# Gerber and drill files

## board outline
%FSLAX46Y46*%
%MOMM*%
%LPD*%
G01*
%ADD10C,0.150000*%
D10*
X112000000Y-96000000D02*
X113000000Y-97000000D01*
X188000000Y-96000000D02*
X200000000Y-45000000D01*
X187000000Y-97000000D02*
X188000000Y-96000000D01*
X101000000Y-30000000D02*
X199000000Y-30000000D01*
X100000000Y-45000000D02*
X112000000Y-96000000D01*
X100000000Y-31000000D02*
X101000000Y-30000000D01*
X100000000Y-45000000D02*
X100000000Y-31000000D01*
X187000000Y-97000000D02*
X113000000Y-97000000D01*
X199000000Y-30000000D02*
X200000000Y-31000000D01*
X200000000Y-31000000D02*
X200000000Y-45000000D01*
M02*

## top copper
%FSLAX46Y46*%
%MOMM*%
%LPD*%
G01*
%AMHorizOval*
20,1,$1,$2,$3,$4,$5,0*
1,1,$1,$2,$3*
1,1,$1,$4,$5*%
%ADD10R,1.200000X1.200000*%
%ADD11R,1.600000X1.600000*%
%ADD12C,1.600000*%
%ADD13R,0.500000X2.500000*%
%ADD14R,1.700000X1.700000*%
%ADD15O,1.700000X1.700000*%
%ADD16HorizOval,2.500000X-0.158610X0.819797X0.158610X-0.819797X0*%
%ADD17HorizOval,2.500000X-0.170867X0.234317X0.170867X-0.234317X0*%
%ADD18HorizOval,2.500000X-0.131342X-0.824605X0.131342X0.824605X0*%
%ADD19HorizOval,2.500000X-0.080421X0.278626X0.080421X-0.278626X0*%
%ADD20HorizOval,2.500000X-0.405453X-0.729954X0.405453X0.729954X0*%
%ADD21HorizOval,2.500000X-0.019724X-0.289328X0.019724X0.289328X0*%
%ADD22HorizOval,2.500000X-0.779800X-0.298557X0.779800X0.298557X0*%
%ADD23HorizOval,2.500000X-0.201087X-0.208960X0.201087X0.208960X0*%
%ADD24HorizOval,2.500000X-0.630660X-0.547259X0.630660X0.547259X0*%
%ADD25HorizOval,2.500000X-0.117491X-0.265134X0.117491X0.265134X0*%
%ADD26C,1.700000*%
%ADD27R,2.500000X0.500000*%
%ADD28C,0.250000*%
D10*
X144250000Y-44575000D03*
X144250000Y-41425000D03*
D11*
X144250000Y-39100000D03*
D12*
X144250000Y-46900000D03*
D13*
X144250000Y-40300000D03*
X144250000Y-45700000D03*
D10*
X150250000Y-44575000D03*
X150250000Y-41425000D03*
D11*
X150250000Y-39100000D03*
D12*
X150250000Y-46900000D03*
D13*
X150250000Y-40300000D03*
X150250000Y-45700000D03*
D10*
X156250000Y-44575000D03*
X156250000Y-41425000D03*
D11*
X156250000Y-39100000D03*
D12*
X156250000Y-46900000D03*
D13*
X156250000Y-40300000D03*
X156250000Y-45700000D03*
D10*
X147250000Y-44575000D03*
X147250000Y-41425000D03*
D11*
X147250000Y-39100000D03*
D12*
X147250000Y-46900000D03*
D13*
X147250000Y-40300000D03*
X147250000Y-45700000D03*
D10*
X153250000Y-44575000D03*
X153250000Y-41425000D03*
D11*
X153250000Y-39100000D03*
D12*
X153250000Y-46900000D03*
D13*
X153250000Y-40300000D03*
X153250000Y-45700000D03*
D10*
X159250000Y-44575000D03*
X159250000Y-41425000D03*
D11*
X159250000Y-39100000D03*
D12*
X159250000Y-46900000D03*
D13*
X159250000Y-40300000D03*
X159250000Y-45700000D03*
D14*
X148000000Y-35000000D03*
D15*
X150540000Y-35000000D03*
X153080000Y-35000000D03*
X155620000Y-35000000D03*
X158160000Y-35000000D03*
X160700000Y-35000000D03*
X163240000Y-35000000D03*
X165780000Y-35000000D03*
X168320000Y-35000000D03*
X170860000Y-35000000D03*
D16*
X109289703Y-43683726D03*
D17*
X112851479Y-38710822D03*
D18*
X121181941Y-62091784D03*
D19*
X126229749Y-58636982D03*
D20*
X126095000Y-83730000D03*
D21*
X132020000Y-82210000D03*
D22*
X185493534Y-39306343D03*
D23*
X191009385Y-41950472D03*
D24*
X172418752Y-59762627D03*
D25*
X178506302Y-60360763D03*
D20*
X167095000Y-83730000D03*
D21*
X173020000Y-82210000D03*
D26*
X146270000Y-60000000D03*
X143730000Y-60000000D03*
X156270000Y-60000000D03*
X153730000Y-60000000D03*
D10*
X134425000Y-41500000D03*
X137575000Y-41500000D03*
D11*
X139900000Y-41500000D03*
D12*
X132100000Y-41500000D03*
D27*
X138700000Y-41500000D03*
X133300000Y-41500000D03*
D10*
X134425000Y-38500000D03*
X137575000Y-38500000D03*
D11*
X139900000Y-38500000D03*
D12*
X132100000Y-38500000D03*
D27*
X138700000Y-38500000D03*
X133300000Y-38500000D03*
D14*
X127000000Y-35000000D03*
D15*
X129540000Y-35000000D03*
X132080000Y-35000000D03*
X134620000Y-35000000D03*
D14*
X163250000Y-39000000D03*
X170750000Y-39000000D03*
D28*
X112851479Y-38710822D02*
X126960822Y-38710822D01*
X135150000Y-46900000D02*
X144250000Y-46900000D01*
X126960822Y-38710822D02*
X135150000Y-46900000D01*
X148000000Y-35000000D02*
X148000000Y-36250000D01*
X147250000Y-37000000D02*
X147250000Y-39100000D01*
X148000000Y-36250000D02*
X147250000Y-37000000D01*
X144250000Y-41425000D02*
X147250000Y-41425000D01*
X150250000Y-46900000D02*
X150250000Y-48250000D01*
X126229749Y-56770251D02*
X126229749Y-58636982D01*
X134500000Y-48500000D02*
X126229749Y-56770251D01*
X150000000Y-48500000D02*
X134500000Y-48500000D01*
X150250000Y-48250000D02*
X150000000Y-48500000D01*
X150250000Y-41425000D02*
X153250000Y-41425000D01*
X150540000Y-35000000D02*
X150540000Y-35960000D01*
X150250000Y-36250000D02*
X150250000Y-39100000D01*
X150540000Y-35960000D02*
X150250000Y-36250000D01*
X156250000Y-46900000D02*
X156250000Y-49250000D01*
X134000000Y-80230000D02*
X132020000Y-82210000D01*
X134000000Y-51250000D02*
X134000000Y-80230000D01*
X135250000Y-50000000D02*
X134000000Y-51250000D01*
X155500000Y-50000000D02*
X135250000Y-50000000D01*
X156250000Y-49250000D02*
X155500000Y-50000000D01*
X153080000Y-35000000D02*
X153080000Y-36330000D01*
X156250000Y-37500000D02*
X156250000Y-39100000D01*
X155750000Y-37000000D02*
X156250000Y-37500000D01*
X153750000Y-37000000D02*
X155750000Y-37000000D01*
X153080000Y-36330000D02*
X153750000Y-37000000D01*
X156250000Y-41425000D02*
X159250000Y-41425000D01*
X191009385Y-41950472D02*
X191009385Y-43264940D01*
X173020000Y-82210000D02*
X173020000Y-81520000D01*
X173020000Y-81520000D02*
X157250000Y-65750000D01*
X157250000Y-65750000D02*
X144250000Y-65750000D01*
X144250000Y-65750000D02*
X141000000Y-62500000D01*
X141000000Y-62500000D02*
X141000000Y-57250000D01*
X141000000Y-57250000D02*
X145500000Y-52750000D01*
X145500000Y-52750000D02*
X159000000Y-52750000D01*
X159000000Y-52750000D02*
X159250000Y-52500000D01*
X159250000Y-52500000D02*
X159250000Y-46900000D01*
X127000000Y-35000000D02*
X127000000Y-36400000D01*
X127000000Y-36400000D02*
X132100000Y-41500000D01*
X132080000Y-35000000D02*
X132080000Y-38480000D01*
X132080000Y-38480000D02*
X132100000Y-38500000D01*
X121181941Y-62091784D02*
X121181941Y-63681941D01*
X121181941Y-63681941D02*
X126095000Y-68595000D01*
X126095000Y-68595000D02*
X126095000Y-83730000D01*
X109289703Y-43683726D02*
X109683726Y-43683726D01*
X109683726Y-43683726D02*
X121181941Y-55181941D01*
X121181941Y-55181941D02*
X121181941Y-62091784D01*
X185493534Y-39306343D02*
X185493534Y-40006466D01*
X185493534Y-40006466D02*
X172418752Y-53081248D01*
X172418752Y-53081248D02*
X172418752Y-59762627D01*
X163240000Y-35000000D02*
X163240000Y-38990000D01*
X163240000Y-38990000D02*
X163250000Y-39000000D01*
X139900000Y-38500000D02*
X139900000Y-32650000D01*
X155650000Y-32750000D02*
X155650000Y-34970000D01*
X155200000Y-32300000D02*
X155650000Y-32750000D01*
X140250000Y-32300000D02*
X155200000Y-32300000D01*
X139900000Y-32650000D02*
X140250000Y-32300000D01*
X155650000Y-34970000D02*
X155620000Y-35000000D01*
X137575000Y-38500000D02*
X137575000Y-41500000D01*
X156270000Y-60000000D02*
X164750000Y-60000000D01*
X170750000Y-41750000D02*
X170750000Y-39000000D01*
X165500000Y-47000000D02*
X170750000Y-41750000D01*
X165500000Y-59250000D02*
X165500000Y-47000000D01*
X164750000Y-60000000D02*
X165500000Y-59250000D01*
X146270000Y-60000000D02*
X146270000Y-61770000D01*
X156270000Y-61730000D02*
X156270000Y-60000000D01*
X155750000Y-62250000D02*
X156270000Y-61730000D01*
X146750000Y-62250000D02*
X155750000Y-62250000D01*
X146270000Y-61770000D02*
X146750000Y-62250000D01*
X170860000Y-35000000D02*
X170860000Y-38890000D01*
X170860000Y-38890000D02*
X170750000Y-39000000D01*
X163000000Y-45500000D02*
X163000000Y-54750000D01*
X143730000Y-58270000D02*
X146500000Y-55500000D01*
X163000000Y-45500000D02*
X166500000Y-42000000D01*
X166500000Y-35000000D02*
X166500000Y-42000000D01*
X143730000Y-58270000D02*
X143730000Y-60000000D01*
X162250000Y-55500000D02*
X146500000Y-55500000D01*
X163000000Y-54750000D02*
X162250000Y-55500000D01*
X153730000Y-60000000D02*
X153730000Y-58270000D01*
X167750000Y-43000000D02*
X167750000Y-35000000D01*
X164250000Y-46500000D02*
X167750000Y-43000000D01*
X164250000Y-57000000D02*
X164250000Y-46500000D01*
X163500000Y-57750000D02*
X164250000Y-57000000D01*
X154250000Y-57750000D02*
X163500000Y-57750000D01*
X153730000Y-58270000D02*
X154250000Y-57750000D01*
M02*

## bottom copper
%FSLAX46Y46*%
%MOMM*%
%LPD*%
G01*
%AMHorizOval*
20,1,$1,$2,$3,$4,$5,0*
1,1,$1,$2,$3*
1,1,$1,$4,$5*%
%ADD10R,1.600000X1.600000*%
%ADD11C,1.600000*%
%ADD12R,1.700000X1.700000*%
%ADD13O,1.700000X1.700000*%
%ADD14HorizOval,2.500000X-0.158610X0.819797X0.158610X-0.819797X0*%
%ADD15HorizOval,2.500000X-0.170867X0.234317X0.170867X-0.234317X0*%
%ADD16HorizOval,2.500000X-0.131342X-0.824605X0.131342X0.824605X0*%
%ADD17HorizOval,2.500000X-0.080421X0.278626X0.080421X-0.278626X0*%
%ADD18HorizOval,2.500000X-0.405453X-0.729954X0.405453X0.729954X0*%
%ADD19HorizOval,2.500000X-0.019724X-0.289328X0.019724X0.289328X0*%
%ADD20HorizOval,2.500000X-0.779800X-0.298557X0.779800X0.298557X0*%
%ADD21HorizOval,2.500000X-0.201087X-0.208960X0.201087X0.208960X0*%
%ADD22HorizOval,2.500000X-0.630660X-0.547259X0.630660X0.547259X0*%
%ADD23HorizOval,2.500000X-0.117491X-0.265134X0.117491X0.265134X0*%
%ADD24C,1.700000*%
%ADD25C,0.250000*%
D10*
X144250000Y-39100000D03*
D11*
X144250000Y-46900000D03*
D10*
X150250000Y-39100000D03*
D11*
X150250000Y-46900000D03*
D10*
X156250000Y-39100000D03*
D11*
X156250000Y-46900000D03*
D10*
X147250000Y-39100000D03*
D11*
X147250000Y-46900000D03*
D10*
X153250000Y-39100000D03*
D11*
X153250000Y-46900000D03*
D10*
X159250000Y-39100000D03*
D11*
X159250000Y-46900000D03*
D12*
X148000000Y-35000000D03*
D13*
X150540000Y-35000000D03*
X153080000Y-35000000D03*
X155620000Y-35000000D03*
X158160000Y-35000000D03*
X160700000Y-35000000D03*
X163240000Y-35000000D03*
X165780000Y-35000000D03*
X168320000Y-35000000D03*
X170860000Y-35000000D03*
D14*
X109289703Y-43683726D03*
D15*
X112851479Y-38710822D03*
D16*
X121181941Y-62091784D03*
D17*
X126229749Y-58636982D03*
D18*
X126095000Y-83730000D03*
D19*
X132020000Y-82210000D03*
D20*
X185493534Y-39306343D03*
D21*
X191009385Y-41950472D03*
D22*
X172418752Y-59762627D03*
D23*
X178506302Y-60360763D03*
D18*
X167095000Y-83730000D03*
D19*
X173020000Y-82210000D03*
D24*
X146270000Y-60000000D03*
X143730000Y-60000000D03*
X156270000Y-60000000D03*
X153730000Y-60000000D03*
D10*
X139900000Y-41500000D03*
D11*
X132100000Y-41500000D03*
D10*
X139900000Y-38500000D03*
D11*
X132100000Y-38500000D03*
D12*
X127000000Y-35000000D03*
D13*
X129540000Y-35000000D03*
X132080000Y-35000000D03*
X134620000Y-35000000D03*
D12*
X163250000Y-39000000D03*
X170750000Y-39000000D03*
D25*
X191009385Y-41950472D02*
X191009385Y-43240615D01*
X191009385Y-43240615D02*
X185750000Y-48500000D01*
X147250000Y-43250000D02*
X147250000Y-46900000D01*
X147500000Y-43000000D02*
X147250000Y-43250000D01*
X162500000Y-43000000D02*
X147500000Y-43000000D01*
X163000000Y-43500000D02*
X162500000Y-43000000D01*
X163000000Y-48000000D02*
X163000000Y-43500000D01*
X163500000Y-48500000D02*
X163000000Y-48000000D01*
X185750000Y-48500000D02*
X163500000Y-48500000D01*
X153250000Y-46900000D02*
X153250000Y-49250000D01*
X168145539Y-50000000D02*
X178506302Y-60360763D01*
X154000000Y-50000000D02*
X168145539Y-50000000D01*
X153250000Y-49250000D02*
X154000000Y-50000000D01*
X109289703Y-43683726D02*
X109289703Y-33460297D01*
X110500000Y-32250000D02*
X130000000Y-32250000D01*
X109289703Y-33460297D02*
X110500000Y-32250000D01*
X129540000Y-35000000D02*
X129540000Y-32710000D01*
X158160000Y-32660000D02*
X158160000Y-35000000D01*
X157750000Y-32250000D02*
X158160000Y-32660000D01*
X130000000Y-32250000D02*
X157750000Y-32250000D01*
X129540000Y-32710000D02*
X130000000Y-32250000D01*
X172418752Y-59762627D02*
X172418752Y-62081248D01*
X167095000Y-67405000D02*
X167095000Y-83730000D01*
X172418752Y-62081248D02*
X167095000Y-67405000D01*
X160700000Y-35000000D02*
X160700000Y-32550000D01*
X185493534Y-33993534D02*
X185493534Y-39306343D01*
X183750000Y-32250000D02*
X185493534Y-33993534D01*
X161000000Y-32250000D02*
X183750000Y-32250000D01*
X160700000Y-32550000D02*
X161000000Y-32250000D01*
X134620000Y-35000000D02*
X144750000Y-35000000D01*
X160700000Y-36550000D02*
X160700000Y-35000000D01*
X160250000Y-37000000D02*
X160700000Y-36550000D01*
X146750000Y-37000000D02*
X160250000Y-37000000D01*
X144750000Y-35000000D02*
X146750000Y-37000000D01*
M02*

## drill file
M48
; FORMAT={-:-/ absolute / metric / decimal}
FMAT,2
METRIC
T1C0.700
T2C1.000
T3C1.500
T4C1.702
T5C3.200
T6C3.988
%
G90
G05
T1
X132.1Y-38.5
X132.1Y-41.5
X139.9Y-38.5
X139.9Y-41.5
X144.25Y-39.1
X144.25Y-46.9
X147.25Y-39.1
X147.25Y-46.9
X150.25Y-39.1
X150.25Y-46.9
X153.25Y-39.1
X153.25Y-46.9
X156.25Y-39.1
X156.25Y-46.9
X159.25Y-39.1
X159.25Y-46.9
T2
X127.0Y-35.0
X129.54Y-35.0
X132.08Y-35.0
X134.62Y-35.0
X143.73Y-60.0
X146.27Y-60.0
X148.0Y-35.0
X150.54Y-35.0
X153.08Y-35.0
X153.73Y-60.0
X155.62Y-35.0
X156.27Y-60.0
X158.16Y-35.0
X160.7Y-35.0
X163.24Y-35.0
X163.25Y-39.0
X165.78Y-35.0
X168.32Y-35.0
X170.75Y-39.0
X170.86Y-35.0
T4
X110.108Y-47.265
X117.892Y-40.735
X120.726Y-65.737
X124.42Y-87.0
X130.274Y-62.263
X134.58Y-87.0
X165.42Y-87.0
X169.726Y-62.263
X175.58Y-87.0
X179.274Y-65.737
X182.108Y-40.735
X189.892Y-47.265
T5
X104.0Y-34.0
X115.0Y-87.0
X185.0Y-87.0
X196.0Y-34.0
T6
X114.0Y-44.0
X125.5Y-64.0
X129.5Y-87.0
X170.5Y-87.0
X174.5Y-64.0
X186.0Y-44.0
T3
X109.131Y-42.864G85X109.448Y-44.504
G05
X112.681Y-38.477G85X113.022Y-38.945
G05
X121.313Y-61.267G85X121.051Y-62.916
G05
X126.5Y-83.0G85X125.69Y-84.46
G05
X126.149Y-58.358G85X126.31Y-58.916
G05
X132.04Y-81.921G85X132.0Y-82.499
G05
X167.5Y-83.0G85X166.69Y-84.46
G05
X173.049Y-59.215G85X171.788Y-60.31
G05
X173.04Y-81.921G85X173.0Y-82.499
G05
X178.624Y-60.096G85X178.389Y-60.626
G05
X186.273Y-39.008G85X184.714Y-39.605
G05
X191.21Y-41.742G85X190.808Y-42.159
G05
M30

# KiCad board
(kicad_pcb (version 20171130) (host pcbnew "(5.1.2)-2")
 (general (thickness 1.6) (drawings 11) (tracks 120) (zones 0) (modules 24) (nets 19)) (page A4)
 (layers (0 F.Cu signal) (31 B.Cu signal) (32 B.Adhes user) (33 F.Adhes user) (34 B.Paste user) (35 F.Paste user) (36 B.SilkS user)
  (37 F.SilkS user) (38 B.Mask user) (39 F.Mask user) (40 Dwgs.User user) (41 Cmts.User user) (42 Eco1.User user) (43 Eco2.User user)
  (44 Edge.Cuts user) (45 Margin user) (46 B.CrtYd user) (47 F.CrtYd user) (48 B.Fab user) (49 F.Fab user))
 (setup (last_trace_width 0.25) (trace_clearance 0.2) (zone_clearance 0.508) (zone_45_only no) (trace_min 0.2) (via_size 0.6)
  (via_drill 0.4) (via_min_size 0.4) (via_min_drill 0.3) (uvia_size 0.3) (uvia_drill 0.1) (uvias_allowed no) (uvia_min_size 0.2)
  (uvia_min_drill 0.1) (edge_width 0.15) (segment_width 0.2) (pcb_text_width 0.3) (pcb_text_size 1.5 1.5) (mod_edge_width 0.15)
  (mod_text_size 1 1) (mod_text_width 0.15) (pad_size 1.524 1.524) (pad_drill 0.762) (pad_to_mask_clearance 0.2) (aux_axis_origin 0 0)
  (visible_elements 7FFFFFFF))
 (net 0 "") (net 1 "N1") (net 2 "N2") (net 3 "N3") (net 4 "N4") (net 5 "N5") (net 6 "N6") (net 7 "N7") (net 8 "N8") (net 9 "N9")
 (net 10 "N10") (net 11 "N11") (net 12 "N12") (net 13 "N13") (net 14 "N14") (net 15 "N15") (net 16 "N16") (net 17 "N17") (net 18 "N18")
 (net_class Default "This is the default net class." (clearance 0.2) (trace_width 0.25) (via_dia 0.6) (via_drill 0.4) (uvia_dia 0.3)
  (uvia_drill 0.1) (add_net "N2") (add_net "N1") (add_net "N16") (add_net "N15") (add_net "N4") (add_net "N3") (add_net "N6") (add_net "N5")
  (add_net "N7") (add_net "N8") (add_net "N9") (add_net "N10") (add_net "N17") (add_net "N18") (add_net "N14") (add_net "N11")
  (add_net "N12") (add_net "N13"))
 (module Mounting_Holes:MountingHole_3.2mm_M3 (layer F.Cu) (at 115 87)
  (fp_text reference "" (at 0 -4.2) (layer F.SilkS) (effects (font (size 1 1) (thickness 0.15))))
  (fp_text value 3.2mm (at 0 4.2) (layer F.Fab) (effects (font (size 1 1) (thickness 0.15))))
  (pad 1 np_thru_hole circle (at 0 0) (size 3.2 3.2) (drill 3.2) (layers *.Cu *.Mask)))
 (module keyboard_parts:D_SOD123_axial (layer F.Cu) (at 144.25 43 270)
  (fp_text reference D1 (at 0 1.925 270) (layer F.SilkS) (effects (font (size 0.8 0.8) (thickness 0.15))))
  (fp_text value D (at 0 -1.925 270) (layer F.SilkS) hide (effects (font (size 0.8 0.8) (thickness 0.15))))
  (pad 2 smd rect (at 1.575 0 270) (size 1.2 1.2) (layers F.Cu F.Paste F.Mask) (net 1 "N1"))
  (pad 1 smd rect (at -1.575 0 270) (size 1.2 1.2) (layers F.Cu F.Paste F.Mask) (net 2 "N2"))
  (pad 1 thru_hole rect (at -3.9 0 270) (size 1.6 1.6) (drill 0.7) (layers *.Cu *.Mask F.SilkS) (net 2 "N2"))
  (pad 2 thru_hole circle (at 3.9 0 270) (size 1.6 1.6) (drill 0.7) (layers *.Cu *.Mask F.SilkS) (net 1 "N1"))
  (pad 1 smd rect (at -2.7 0 270) (size 2.5 0.5) (layers F.Cu) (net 2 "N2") (solder_mask_margin -999))
  (pad 2 smd rect (at 2.7 0 270) (size 2.5 0.5) (layers F.Cu) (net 1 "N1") (solder_mask_margin -999)))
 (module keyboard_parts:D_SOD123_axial (layer F.Cu) (at 150.25 43 270)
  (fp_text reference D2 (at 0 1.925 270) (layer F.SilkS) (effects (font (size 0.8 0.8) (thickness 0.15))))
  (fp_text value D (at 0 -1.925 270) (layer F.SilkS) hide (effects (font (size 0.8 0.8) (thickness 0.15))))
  (pad 2 smd rect (at 1.575 0 270) (size 1.2 1.2) (layers F.Cu F.Paste F.Mask) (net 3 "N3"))
  (pad 1 smd rect (at -1.575 0 270) (size 1.2 1.2) (layers F.Cu F.Paste F.Mask) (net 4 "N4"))
  (pad 1 thru_hole rect (at -3.9 0 270) (size 1.6 1.6) (drill 0.7) (layers *.Cu *.Mask F.SilkS) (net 4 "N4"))
  (pad 2 thru_hole circle (at 3.9 0 270) (size 1.6 1.6) (drill 0.7) (layers *.Cu *.Mask F.SilkS) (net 3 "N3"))
  (pad 1 smd rect (at -2.7 0 270) (size 2.5 0.5) (layers F.Cu) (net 4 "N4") (solder_mask_margin -999))
  (pad 2 smd rect (at 2.7 0 270) (size 2.5 0.5) (layers F.Cu) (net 3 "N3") (solder_mask_margin -999)))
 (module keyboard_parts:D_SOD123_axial (layer F.Cu) (at 156.25 43 270)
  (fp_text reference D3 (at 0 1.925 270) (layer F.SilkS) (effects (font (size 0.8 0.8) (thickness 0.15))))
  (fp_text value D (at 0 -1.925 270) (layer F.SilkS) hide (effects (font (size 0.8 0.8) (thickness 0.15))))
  (pad 2 smd rect (at 1.575 0 270) (size 1.2 1.2) (layers F.Cu F.Paste F.Mask) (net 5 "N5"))
  (pad 1 smd rect (at -1.575 0 270) (size 1.2 1.2) (layers F.Cu F.Paste F.Mask) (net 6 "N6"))
  (pad 1 thru_hole rect (at -3.9 0 270) (size 1.6 1.6) (drill 0.7) (layers *.Cu *.Mask F.SilkS) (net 6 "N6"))
  (pad 2 thru_hole circle (at 3.9 0 270) (size 1.6 1.6) (drill 0.7) (layers *.Cu *.Mask F.SilkS) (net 5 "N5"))
  (pad 1 smd rect (at -2.7 0 270) (size 2.5 0.5) (layers F.Cu) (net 6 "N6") (solder_mask_margin -999))
  (pad 2 smd rect (at 2.7 0 270) (size 2.5 0.5) (layers F.Cu) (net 5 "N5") (solder_mask_margin -999)))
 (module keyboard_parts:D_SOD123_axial (layer F.Cu) (at 147.25 43 270)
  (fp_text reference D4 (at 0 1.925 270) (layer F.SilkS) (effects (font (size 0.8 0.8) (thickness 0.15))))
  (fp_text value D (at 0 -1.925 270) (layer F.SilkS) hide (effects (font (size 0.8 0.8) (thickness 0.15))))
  (pad 2 smd rect (at 1.575 0 270) (size 1.2 1.2) (layers F.Cu F.Paste F.Mask) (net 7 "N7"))
  (pad 1 smd rect (at -1.575 0 270) (size 1.2 1.2) (layers F.Cu F.Paste F.Mask) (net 2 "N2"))
  (pad 1 thru_hole rect (at -3.9 0 270) (size 1.6 1.6) (drill 0.7) (layers *.Cu *.Mask F.SilkS) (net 2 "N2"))
  (pad 2 thru_hole circle (at 3.9 0 270) (size 1.6 1.6) (drill 0.7) (layers *.Cu *.Mask F.SilkS) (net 7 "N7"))
  (pad 1 smd rect (at -2.7 0 270) (size 2.5 0.5) (layers F.Cu) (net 2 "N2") (solder_mask_margin -999))
  (pad 2 smd rect (at 2.7 0 270) (size 2.5 0.5) (layers F.Cu) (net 7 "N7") (solder_mask_margin -999)))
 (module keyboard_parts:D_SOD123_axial (layer F.Cu) (at 153.25 43 270)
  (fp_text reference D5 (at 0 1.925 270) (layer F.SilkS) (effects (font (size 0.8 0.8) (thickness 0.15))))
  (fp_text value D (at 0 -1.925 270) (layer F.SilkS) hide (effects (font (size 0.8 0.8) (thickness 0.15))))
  (pad 2 smd rect (at 1.575 0 270) (size 1.2 1.2) (layers F.Cu F.Paste F.Mask) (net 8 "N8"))
  (pad 1 smd rect (at -1.575 0 270) (size 1.2 1.2) (layers F.Cu F.Paste F.Mask) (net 4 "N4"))
  (pad 1 thru_hole rect (at -3.9 0 270) (size 1.6 1.6) (drill 0.7) (layers *.Cu *.Mask F.SilkS) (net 4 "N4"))
  (pad 2 thru_hole circle (at 3.9 0 270) (size 1.6 1.6) (drill 0.7) (layers *.Cu *.Mask F.SilkS) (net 8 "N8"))
  (pad 1 smd rect (at -2.7 0 270) (size 2.5 0.5) (layers F.Cu) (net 4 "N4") (solder_mask_margin -999))
  (pad 2 smd rect (at 2.7 0 270) (size 2.5 0.5) (layers F.Cu) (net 8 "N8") (solder_mask_margin -999)))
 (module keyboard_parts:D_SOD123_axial (layer F.Cu) (at 159.25 43 270)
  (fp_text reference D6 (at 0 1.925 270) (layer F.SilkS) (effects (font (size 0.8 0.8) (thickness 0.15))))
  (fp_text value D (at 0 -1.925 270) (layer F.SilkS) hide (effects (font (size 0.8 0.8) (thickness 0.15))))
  (pad 2 smd rect (at 1.575 0 270) (size 1.2 1.2) (layers F.Cu F.Paste F.Mask) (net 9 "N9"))
  (pad 1 smd rect (at -1.575 0 270) (size 1.2 1.2) (layers F.Cu F.Paste F.Mask) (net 6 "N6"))
  (pad 1 thru_hole rect (at -3.9 0 270) (size 1.6 1.6) (drill 0.7) (layers *.Cu *.Mask F.SilkS) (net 6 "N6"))
  (pad 2 thru_hole circle (at 3.9 0 270) (size 1.6 1.6) (drill 0.7) (layers *.Cu *.Mask F.SilkS) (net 9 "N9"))
  (pad 1 smd rect (at -2.7 0 270) (size 2.5 0.5) (layers F.Cu) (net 6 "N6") (solder_mask_margin -999))
  (pad 2 smd rect (at 2.7 0 270) (size 2.5 0.5) (layers F.Cu) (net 9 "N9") (solder_mask_margin -999)))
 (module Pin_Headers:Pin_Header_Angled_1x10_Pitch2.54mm (layer F.Cu) (at 148 35 90)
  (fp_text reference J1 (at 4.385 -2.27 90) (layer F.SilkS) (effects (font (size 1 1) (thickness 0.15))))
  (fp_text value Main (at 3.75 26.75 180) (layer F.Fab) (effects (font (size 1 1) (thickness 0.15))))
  (pad 1 thru_hole rect (at 0 0 90) (size 1.7 1.7) (drill 1) (layers *.Cu *.Mask) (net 2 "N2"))
  (pad 2 thru_hole oval (at 0 2.54 90) (size 1.7 1.7) (drill 1) (layers *.Cu *.Mask) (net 4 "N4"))
  (pad 3 thru_hole oval (at 0 5.08 90) (size 1.7 1.7) (drill 1) (layers *.Cu *.Mask) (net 6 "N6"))
  (pad 4 thru_hole oval (at 0 7.62 90) (size 1.7 1.7) (drill 1) (layers *.Cu *.Mask) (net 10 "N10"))
  (pad 5 thru_hole oval (at 0 10.16 90) (size 1.7 1.7) (drill 1) (layers *.Cu *.Mask) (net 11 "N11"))
  (pad 6 thru_hole oval (at 0 12.7 90) (size 1.7 1.7) (drill 1) (layers *.Cu *.Mask) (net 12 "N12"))
  (pad 7 thru_hole oval (at 0 15.24 90) (size 1.7 1.7) (drill 1) (layers *.Cu *.Mask) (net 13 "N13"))
  (pad 8 thru_hole oval (at 0 17.78 90) (size 1.7 1.7) (drill 1) (layers *.Cu *.Mask) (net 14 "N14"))
  (pad 9 thru_hole oval (at 0 20.32 90) (size 1.7 1.7) (drill 1) (layers *.Cu *.Mask) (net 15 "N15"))
  (pad 10 thru_hole oval (at 0 22.86 90) (size 1.7 1.7) (drill 1) (layers *.Cu *.Mask) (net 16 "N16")))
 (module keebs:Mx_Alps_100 (layer F.Cu) (at 114 44 40)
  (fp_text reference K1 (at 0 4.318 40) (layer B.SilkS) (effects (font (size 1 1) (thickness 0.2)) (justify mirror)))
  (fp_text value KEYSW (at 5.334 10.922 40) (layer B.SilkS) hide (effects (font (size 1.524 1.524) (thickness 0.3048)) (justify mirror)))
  (pad HOLE np_thru_hole circle (at 0 0 40) (size 3.9878 3.9878) (drill 3.9878) (layers *.Cu))
  (pad HOLE np_thru_hole circle (at -5.08 0 40) (size 1.7018 1.7018) (drill 1.7018) (layers *.Cu))
  (pad HOLE np_thru_hole circle (at 5.08 0 40) (size 1.7018 1.7018) (drill 1.7018) (layers *.Cu))
  (pad 1 thru_hole oval (at -3.405 -3.27 10.95) (size 2.5 4.17) (drill oval 1.5 3.17) (layers *.Cu *.Mask F.SilkS) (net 11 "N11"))
  (pad 2 thru_hole oval (at 2.52 -4.79 36.1) (size 2.5 3.08) (drill oval 1.5 2.08) (layers *.Cu *.Mask F.SilkS) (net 1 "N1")))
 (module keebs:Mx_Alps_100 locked (layer F.Cu) (at 125.5 64 20)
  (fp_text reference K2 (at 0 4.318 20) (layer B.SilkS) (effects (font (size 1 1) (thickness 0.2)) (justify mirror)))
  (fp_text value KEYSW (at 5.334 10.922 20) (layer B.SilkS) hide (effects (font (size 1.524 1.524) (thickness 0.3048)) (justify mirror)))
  (pad HOLE np_thru_hole circle (at 0 0 20) (size 3.9878 3.9878) (drill 3.9878) (layers *.Cu))
  (pad HOLE np_thru_hole circle (at -5.08 0 20) (size 1.7018 1.7018) (drill 1.7018) (layers *.Cu))
  (pad HOLE np_thru_hole circle (at 5.08 0 20) (size 1.7018 1.7018) (drill 1.7018) (layers *.Cu))
  (pad 1 thru_hole oval (at -3.405 -3.27 350.95) (size 2.5 4.17) (drill oval 1.5 3.17) (layers *.Cu *.Mask F.SilkS) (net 11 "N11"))
  (pad 2 thru_hole oval (at 2.52 -4.79 16.1) (size 2.5 3.08) (drill oval 1.5 2.08) (layers *.Cu *.Mask F.SilkS) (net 3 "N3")))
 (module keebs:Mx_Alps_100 (layer F.Cu) (at 129.5 87)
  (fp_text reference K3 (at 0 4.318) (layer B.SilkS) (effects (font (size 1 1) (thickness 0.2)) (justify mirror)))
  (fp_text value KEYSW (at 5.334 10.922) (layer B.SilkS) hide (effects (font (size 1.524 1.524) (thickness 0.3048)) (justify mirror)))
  (pad HOLE np_thru_hole circle (at 0 0) (size 3.9878 3.9878) (drill 3.9878) (layers *.Cu))
  (pad HOLE np_thru_hole circle (at -5.08 0) (size 1.7018 1.7018) (drill 1.7018) (layers *.Cu))
  (pad HOLE np_thru_hole circle (at 5.08 0) (size 1.7018 1.7018) (drill 1.7018) (layers *.Cu))
  (pad 1 thru_hole oval (at -3.405 -3.27 330.95) (size 2.5 4.17) (drill oval 1.5 3.17) (layers *.Cu *.Mask F.SilkS) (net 11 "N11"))
  (pad 2 thru_hole oval (at 2.52 -4.79 356.1) (size 2.5 3.08) (drill oval 1.5 2.08) (layers *.Cu *.Mask F.SilkS) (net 5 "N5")))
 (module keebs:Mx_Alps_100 (layer F.Cu) (at 186 44 320)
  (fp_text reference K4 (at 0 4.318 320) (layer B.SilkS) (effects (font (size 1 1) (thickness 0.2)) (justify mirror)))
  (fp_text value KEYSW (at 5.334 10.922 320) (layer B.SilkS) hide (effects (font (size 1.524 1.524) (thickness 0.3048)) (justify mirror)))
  (pad HOLE np_thru_hole circle (at 0 0 320) (size 3.9878 3.9878) (drill 3.9878) (layers *.Cu))
  (pad HOLE np_thru_hole circle (at -5.08 0 320) (size 1.7018 1.7018) (drill 1.7018) (layers *.Cu))
  (pad HOLE np_thru_hole circle (at 5.08 0 320) (size 1.7018 1.7018) (drill 1.7018) (layers *.Cu))
  (pad 1 thru_hole oval (at -3.405 -3.27 290.95) (size 2.5 4.17) (drill oval 1.5 3.17) (layers *.Cu *.Mask F.SilkS) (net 12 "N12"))
  (pad 2 thru_hole oval (at 2.52 -4.79 316.1) (size 2.5 3.08) (drill oval 1.5 2.08) (layers *.Cu *.Mask F.SilkS) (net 7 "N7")))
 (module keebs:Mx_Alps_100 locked (layer F.Cu) (at 174.5 64 340)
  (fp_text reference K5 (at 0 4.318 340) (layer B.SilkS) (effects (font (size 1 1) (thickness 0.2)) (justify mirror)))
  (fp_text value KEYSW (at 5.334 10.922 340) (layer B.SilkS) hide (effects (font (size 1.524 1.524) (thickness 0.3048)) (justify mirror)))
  (pad HOLE np_thru_hole circle (at 0 0 340) (size 3.9878 3.9878) (drill 3.9878) (layers *.Cu))
  (pad HOLE np_thru_hole circle (at -5.08 0 340) (size 1.7018 1.7018) (drill 1.7018) (layers *.Cu))
  (pad HOLE np_thru_hole circle (at 5.08 0 340) (size 1.7018 1.7018) (drill 1.7018) (layers *.Cu))
  (pad 1 thru_hole oval (at -3.405 -3.27 310.95) (size 2.5 4.17) (drill oval 1.5 3.17) (layers *.Cu *.Mask F.SilkS) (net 12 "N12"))
  (pad 2 thru_hole oval (at 2.52 -4.79 336.1) (size 2.5 3.08) (drill oval 1.5 2.08) (layers *.Cu *.Mask F.SilkS) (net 8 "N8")))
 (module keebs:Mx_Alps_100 (layer F.Cu) (at 170.5 87)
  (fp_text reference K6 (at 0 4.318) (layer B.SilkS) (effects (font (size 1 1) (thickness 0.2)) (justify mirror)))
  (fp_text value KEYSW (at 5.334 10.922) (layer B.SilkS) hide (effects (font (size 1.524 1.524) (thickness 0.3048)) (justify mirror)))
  (pad HOLE np_thru_hole circle (at 0 0) (size 3.9878 3.9878) (drill 3.9878) (layers *.Cu))
  (pad HOLE np_thru_hole circle (at -5.08 0) (size 1.7018 1.7018) (drill 1.7018) (layers *.Cu))
  (pad HOLE np_thru_hole circle (at 5.08 0) (size 1.7018 1.7018) (drill 1.7018) (layers *.Cu))
  (pad 1 thru_hole oval (at -3.405 -3.27 330.95) (size 2.5 4.17) (drill oval 1.5 3.17) (layers *.Cu *.Mask F.SilkS) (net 12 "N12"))
  (pad 2 thru_hole oval (at 2.52 -4.79 356.1) (size 2.5 3.08) (drill oval 1.5 2.08) (layers *.Cu *.Mask F.SilkS) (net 9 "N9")))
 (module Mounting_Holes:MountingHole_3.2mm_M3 (layer F.Cu) (at 196 34)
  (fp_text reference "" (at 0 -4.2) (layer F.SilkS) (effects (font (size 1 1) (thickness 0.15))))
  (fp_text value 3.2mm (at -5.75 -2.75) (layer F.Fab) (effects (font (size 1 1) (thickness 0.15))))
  (pad 1 np_thru_hole circle (at 0 0) (size 3.2 3.2) (drill 3.2) (layers *.Cu *.Mask)))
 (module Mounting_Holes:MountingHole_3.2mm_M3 (layer F.Cu) (at 185 87)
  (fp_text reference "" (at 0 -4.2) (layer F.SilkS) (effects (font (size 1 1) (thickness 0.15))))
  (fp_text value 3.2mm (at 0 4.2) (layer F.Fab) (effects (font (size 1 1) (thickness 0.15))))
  (pad 1 np_thru_hole circle (at 0 0) (size 3.2 3.2) (drill 3.2) (layers *.Cu *.Mask)))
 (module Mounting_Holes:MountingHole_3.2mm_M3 (layer F.Cu) (at 104 34)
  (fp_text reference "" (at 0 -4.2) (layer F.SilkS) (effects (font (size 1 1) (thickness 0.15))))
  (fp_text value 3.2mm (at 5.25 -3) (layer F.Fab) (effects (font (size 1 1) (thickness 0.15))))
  (pad 1 np_thru_hole circle (at 0 0) (size 3.2 3.2) (drill 3.2) (layers *.Cu *.Mask)))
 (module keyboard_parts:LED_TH (layer F.Cu) (at 145 60 180)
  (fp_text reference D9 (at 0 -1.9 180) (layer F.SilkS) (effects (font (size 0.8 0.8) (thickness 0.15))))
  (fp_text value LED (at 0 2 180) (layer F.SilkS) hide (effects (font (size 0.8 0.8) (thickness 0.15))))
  (pad 1 thru_hole circle (at -1.27 0 180) (size 1.7 1.7) (drill 1) (layers *.Cu *.Mask F.SilkS) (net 16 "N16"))
  (pad 2 thru_hole circle (at 1.27 0 180) (size 1.7 1.7) (drill 1) (layers *.Cu *.Mask F.SilkS) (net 14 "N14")))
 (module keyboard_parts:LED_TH (layer F.Cu) (at 155 60 180)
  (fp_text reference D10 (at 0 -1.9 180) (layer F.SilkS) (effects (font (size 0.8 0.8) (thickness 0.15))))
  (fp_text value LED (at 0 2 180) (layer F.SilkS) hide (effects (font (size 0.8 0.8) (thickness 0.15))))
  (pad 1 thru_hole circle (at -1.27 0 180) (size 1.7 1.7) (drill 1) (layers *.Cu *.Mask F.SilkS) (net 16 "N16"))
  (pad 2 thru_hole circle (at 1.27 0 180) (size 1.7 1.7) (drill 1) (layers *.Cu *.Mask F.SilkS) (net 15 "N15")))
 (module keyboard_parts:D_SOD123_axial (layer F.Cu) (at 136 41.5 180)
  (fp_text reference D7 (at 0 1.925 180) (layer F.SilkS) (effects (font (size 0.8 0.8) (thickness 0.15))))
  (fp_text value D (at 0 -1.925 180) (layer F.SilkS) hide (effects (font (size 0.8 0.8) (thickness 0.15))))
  (pad 2 smd rect (at 1.575 0 180) (size 1.2 1.2) (layers F.Cu F.Paste F.Mask) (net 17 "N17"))
  (pad 1 smd rect (at -1.575 0 180) (size 1.2 1.2) (layers F.Cu F.Paste F.Mask) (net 10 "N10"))
  (pad 1 thru_hole rect (at -3.9 0 180) (size 1.6 1.6) (drill 0.7) (layers *.Cu *.Mask F.SilkS) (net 10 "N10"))
  (pad 2 thru_hole circle (at 3.9 0 180) (size 1.6 1.6) (drill 0.7) (layers *.Cu *.Mask F.SilkS) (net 17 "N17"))
  (pad 1 smd rect (at -2.7 0 180) (size 2.5 0.5) (layers F.Cu) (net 10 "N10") (solder_mask_margin -999))
  (pad 2 smd rect (at 2.7 0 180) (size 2.5 0.5) (layers F.Cu) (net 17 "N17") (solder_mask_margin -999)))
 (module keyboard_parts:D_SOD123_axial (layer F.Cu) (at 136 38.5 180)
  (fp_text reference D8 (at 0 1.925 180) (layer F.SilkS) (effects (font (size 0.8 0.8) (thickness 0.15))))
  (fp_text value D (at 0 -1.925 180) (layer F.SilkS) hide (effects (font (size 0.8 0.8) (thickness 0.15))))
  (pad 2 smd rect (at 1.575 0 180) (size 1.2 1.2) (layers F.Cu F.Paste F.Mask) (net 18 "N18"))
  (pad 1 smd rect (at -1.575 0 180) (size 1.2 1.2) (layers F.Cu F.Paste F.Mask) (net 10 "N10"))
  (pad 1 thru_hole rect (at -3.9 0 180) (size 1.6 1.6) (drill 0.7) (layers *.Cu *.Mask F.SilkS) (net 10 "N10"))
  (pad 2 thru_hole circle (at 3.9 0 180) (size 1.6 1.6) (drill 0.7) (layers *.Cu *.Mask F.SilkS) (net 18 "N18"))
  (pad 1 smd rect (at -2.7 0 180) (size 2.5 0.5) (layers F.Cu) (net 10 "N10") (solder_mask_margin -999))
  (pad 2 smd rect (at 2.7 0 180) (size 2.5 0.5) (layers F.Cu) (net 18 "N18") (solder_mask_margin -999)))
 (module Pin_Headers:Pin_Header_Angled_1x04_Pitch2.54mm (layer F.Cu) (at 127 35 90)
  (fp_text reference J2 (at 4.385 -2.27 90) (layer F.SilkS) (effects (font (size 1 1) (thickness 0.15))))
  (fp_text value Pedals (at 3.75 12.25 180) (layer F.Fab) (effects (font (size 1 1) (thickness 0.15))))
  (pad 1 thru_hole rect (at 0 0 90) (size 1.7 1.7) (drill 1) (layers *.Cu *.Mask) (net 17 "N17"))
  (pad 2 thru_hole oval (at 0 2.54 90) (size 1.7 1.7) (drill 1) (layers *.Cu *.Mask) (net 11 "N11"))
  (pad 3 thru_hole oval (at 0 5.08 90) (size 1.7 1.7) (drill 1) (layers *.Cu *.Mask) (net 18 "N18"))
  (pad 4 thru_hole oval (at 0 7.62 90) (size 1.7 1.7) (drill 1) (layers *.Cu *.Mask) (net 12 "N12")))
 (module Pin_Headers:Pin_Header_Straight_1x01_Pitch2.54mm (layer F.Cu) (at 163.25 39)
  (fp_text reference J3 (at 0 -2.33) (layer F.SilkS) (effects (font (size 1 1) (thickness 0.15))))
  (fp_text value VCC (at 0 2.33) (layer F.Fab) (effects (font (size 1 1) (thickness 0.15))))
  (pad 1 thru_hole rect (at 0 0) (size 1.7 1.7) (drill 1) (layers *.Cu *.Mask) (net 13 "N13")))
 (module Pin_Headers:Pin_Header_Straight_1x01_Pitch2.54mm (layer F.Cu) (at 170.75 39)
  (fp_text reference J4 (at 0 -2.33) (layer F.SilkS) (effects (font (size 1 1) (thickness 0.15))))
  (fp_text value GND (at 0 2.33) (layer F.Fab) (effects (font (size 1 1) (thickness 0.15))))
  (pad 1 thru_hole rect (at 0 0) (size 1.7 1.7) (drill 1) (layers *.Cu *.Mask) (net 16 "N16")))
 (gr_line (start 112 96) (end 113 97) (angle 90) (layer Edge.Cuts) (width 0.15))
 (gr_line (start 188 96) (end 200 45) (angle 90) (layer Edge.Cuts) (width 0.15))
 (gr_line (start 187 97) (end 188 96) (angle 90) (layer Edge.Cuts) (width 0.15))
 (gr_line (start 101 30) (end 199 30) (angle 90) (layer Edge.Cuts) (width 0.15))
 (gr_line (start 100 45) (end 112 96) (angle 90) (layer Edge.Cuts) (width 0.15))
 (gr_line (start 100 31) (end 101 30) (angle 90) (layer Edge.Cuts) (width 0.15))
 (gr_line (start 100 45) (end 100 31) (angle 90) (layer Edge.Cuts) (width 0.15))
 (gr_line (start 187 97) (end 113 97) (angle 90) (layer Edge.Cuts) (width 0.15))
 (gr_line (start 199 30) (end 200 31) (angle 90) (layer Edge.Cuts) (width 0.15))
 (gr_line (start 200 31) (end 200 45) (angle 90) (layer Edge.Cuts) (width 0.15))
 (segment (start 112.851479 38.710822) (end 126.960822 38.710822) (width 0.25) (layer F.Cu) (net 1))
 (segment (start 135.15 46.9) (end 144.25 46.9) (width 0.25) (layer F.Cu) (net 1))
 (segment (start 126.960822 38.710822) (end 135.15 46.9) (width 0.25) (layer F.Cu) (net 1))
 (segment (start 148 35) (end 148 36.25) (width 0.25) (layer F.Cu) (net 2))
 (segment (start 147.25 37) (end 147.25 39.1) (width 0.25) (layer F.Cu) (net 2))
 (segment (start 148 36.25) (end 147.25 37) (width 0.25) (layer F.Cu) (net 2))
 (segment (start 144.25 41.425) (end 147.25 41.425) (width 0.25) (layer F.Cu) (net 2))
 (segment (start 150.25 46.9) (end 150.25 48.25) (width 0.25) (layer F.Cu) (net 3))
 (segment (start 126.229749 56.770251) (end 126.229749 58.636982) (width 0.25) (layer F.Cu) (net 3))
 (segment (start 134.5 48.5) (end 126.229749 56.770251) (width 0.25) (layer F.Cu) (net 3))
 (segment (start 150 48.5) (end 134.5 48.5) (width 0.25) (layer F.Cu) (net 3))
 (segment (start 150.25 48.25) (end 150 48.5) (width 0.25) (layer F.Cu) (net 3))
 (segment (start 150.25 41.425) (end 153.25 41.425) (width 0.25) (layer F.Cu) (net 4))
 (segment (start 150.54 35) (end 150.54 35.96) (width 0.25) (layer F.Cu) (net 4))
 (segment (start 150.25 36.25) (end 150.25 39.1) (width 0.25) (layer F.Cu) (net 4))
 (segment (start 150.54 35.96) (end 150.25 36.25) (width 0.25) (layer F.Cu) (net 4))
 (segment (start 156.25 46.9) (end 156.25 49.25) (width 0.25) (layer F.Cu) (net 5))
 (segment (start 134 80.23) (end 132.02 82.21) (width 0.25) (layer F.Cu) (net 5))
 (segment (start 134 51.25) (end 134 80.23) (width 0.25) (layer F.Cu) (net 5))
 (segment (start 135.25 50) (end 134 51.25) (width 0.25) (layer F.Cu) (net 5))
 (segment (start 155.5 50) (end 135.25 50) (width 0.25) (layer F.Cu) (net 5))
 (segment (start 156.25 49.25) (end 155.5 50) (width 0.25) (layer F.Cu) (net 5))
 (segment (start 153.08 35) (end 153.08 36.33) (width 0.25) (layer F.Cu) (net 6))
 (segment (start 156.25 37.5) (end 156.25 39.1) (width 0.25) (layer F.Cu) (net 6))
 (segment (start 155.75 37) (end 156.25 37.5) (width 0.25) (layer F.Cu) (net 6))
 (segment (start 153.75 37) (end 155.75 37) (width 0.25) (layer F.Cu) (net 6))
 (segment (start 153.08 36.33) (end 153.75 37) (width 0.25) (layer F.Cu) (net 6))
 (segment (start 156.25 41.425) (end 159.25 41.425) (width 0.25) (layer F.Cu) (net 6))
 (segment (start 191.009385 41.950472) (end 191.009385 43.240615) (width 0.25) (layer B.Cu) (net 7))
 (segment (start 191.009385 43.240615) (end 185.75 48.5) (width 0.25) (layer B.Cu) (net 7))
 (segment (start 147.25 43.25) (end 147.25 46.9) (width 0.25) (layer B.Cu) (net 7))
 (segment (start 147.5 43) (end 147.25 43.25) (width 0.25) (layer B.Cu) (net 7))
 (segment (start 162.5 43) (end 147.5 43) (width 0.25) (layer B.Cu) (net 7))
 (segment (start 163 43.5) (end 162.5 43) (width 0.25) (layer B.Cu) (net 7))
 (segment (start 163 48) (end 163 43.5) (width 0.25) (layer B.Cu) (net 7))
 (segment (start 163.5 48.5) (end 163 48) (width 0.25) (layer B.Cu) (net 7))
 (segment (start 185.75 48.5) (end 163.5 48.5) (width 0.25) (layer B.Cu) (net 7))
 (segment (start 191.009385 41.950472) (end 191.009385 43.26494) (width 0.25) (layer F.Cu) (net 7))
 (segment (start 153.25 46.9) (end 153.25 49.25) (width 0.25) (layer B.Cu) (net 8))
 (segment (start 168.145539 50) (end 178.506302 60.360763) (width 0.25) (layer B.Cu) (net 8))
 (segment (start 154 50) (end 168.145539 50) (width 0.25) (layer B.Cu) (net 8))
 (segment (start 153.25 49.25) (end 154 50) (width 0.25) (layer B.Cu) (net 8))
 (segment (start 173.02 82.21) (end 173.02 81.52) (width 0.25) (layer F.Cu) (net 9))
 (segment (start 173.02 81.52) (end 157.25 65.75) (width 0.25) (layer F.Cu) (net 9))
 (segment (start 157.25 65.75) (end 144.25 65.75) (width 0.25) (layer F.Cu) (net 9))
 (segment (start 144.25 65.75) (end 141 62.5) (width 0.25) (layer F.Cu) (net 9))
 (segment (start 141 62.5) (end 141 57.25) (width 0.25) (layer F.Cu) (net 9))
 (segment (start 141 57.25) (end 145.5 52.75) (width 0.25) (layer F.Cu) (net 9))
 (segment (start 145.5 52.75) (end 159 52.75) (width 0.25) (layer F.Cu) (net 9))
 (segment (start 159 52.75) (end 159.25 52.5) (width 0.25) (layer F.Cu) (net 9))
 (segment (start 159.25 52.5) (end 159.25 46.9) (width 0.25) (layer F.Cu) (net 9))
 (segment (start 127 35) (end 127 36.4) (width 0.25) (layer F.Cu) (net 17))
 (segment (start 127 36.4) (end 132.1 41.5) (width 0.25) (layer F.Cu) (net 17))
 (segment (start 132.08 35) (end 132.08 38.48) (width 0.25) (layer F.Cu) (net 18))
 (segment (start 132.08 38.48) (end 132.1 38.5) (width 0.25) (layer F.Cu) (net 18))
 (segment (start 121.181941 62.091784) (end 121.181941 63.681941) (width 0.25) (layer F.Cu) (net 11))
 (segment (start 121.181941 63.681941) (end 126.095 68.595) (width 0.25) (layer F.Cu) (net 11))
 (segment (start 126.095 68.595) (end 126.095 83.73) (width 0.25) (layer F.Cu) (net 11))
 (segment (start 109.289703 43.683726) (end 109.683726 43.683726) (width 0.25) (layer F.Cu) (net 11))
 (segment (start 109.683726 43.683726) (end 121.181941 55.181941) (width 0.25) (layer F.Cu) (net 11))
 (segment (start 121.181941 55.181941) (end 121.181941 62.091784) (width 0.25) (layer F.Cu) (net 11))
 (segment (start 109.289703 43.683726) (end 109.289703 33.460297) (width 0.25) (layer B.Cu) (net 11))
 (segment (start 110.5 32.25) (end 130 32.25) (width 0.25) (layer B.Cu) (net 11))
 (segment (start 109.289703 33.460297) (end 110.5 32.25) (width 0.25) (layer B.Cu) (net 11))
 (segment (start 129.54 35) (end 129.54 32.71) (width 0.25) (layer B.Cu) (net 11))
 (segment (start 158.16 32.66) (end 158.16 35) (width 0.25) (layer B.Cu) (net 11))
 (segment (start 157.75 32.25) (end 158.16 32.66) (width 0.25) (layer B.Cu) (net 11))
 (segment (start 130 32.25) (end 157.75 32.25) (width 0.25) (layer B.Cu) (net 11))
 (segment (start 129.54 32.71) (end 130 32.25) (width 0.25) (layer B.Cu) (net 11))
 (segment (start 172.418752 59.762627) (end 172.418752 62.081248) (width 0.25) (layer B.Cu) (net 12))
 (segment (start 167.095 67.405) (end 167.095 83.73) (width 0.25) (layer B.Cu) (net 12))
 (segment (start 172.418752 62.081248) (end 167.095 67.405) (width 0.25) (layer B.Cu) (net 12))
 (segment (start 185.493534 39.306343) (end 185.493534 40.006466) (width 0.25) (layer F.Cu) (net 12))
 (segment (start 185.493534 40.006466) (end 172.418752 53.081248) (width 0.25) (layer F.Cu) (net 12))
 (segment (start 172.418752 53.081248) (end 172.418752 59.762627) (width 0.25) (layer F.Cu) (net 12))
 (segment (start 160.7 35) (end 160.7 32.55) (width 0.25) (layer B.Cu) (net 12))
 (segment (start 185.493534 33.993534) (end 185.493534 39.306343) (width 0.25) (layer B.Cu) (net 12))
 (segment (start 183.75 32.25) (end 185.493534 33.993534) (width 0.25) (layer B.Cu) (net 12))
 (segment (start 161 32.25) (end 183.75 32.25) (width 0.25) (layer B.Cu) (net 12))
 (segment (start 160.7 32.55) (end 161 32.25) (width 0.25) (layer B.Cu) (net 12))
 (segment (start 134.62 35) (end 144.75 35) (width 0.25) (layer B.Cu) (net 12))
 (segment (start 160.7 36.55) (end 160.7 35) (width 0.25) (layer B.Cu) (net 12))
 (segment (start 160.25 37) (end 160.7 36.55) (width 0.25) (layer B.Cu) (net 12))
 (segment (start 146.75 37) (end 160.25 37) (width 0.25) (layer B.Cu) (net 12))
 (segment (start 144.75 35) (end 146.75 37) (width 0.25) (layer B.Cu) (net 12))
 (segment (start 163.24 35) (end 163.24 38.99) (width 0.25) (layer F.Cu) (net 13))
 (segment (start 163.24 38.99) (end 163.25 39) (width 0.25) (layer F.Cu) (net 13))
 (segment (start 139.9 38.5) (end 139.9 32.65) (width 0.25) (layer F.Cu) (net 10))
 (segment (start 155.65 32.75) (end 155.65 34.97) (width 0.25) (layer F.Cu) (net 10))
 (segment (start 155.2 32.3) (end 155.65 32.75) (width 0.25) (layer F.Cu) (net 10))
 (segment (start 140.25 32.3) (end 155.2 32.3) (width 0.25) (layer F.Cu) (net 10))
 (segment (start 139.9 32.65) (end 140.25 32.3) (width 0.25) (layer F.Cu) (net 10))
 (segment (start 155.65 34.97) (end 155.62 35) (width 0.25) (layer F.Cu) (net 10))
 (segment (start 137.575 38.5) (end 137.575 41.5) (width 0.25) (layer F.Cu) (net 10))
 (segment (start 156.27 60) (end 164.75 60) (width 0.25) (layer F.Cu) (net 16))
 (segment (start 170.75 41.75) (end 170.75 39) (width 0.25) (layer F.Cu) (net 16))
 (segment (start 165.5 47) (end 170.75 41.75) (width 0.25) (layer F.Cu) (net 16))
 (segment (start 165.5 59.25) (end 165.5 47) (width 0.25) (layer F.Cu) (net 16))
 (segment (start 164.75 60) (end 165.5 59.25) (width 0.25) (layer F.Cu) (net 16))
 (segment (start 146.27 60) (end 146.27 61.77) (width 0.25) (layer F.Cu) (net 16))
 (segment (start 156.27 61.73) (end 156.27 60) (width 0.25) (layer F.Cu) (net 16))
 (segment (start 155.75 62.25) (end 156.27 61.73) (width 0.25) (layer F.Cu) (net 16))
 (segment (start 146.75 62.25) (end 155.75 62.25) (width 0.25) (layer F.Cu) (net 16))
 (segment (start 146.27 61.77) (end 146.75 62.25) (width 0.25) (layer F.Cu) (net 16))
 (segment (start 170.86 35) (end 170.86 38.89) (width 0.25) (layer F.Cu) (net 16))
 (segment (start 170.86 38.89) (end 170.75 39) (width 0.25) (layer F.Cu) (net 16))
 (segment (start 163 45.5) (end 163 54.75) (width 0.25) (layer F.Cu) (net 14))
 (segment (start 143.73 58.27) (end 146.5 55.5) (width 0.25) (layer F.Cu) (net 14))
 (segment (start 163 45.5) (end 166.5 42) (width 0.25) (layer F.Cu) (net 14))
 (segment (start 166.5 35) (end 166.5 42) (width 0.25) (layer F.Cu) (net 14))
 (segment (start 143.73 58.27) (end 143.73 60) (width 0.25) (layer F.Cu) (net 14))
 (segment (start 162.25 55.5) (end 146.5 55.5) (width 0.25) (layer F.Cu) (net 14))
 (segment (start 163 54.75) (end 162.25 55.5) (width 0.25) (layer F.Cu) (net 14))
 (segment (start 153.73 60) (end 153.73 58.27) (width 0.25) (layer F.Cu) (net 15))
 (segment (start 167.75 43) (end 167.75 35) (width 0.25) (layer F.Cu) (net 15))
 (segment (start 164.25 46.5) (end 167.75 43) (width 0.25) (layer F.Cu) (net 15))
 (segment (start 164.25 57) (end 164.25 46.5) (width 0.25) (layer F.Cu) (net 15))
 (segment (start 163.5 57.75) (end 164.25 57) (width 0.25) (layer F.Cu) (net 15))
 (segment (start 154.25 57.75) (end 163.5 57.75) (width 0.25) (layer F.Cu) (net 15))
 (segment (start 153.73 58.27) (end 154.25 57.75) (width 0.25) (layer F.Cu) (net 15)))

